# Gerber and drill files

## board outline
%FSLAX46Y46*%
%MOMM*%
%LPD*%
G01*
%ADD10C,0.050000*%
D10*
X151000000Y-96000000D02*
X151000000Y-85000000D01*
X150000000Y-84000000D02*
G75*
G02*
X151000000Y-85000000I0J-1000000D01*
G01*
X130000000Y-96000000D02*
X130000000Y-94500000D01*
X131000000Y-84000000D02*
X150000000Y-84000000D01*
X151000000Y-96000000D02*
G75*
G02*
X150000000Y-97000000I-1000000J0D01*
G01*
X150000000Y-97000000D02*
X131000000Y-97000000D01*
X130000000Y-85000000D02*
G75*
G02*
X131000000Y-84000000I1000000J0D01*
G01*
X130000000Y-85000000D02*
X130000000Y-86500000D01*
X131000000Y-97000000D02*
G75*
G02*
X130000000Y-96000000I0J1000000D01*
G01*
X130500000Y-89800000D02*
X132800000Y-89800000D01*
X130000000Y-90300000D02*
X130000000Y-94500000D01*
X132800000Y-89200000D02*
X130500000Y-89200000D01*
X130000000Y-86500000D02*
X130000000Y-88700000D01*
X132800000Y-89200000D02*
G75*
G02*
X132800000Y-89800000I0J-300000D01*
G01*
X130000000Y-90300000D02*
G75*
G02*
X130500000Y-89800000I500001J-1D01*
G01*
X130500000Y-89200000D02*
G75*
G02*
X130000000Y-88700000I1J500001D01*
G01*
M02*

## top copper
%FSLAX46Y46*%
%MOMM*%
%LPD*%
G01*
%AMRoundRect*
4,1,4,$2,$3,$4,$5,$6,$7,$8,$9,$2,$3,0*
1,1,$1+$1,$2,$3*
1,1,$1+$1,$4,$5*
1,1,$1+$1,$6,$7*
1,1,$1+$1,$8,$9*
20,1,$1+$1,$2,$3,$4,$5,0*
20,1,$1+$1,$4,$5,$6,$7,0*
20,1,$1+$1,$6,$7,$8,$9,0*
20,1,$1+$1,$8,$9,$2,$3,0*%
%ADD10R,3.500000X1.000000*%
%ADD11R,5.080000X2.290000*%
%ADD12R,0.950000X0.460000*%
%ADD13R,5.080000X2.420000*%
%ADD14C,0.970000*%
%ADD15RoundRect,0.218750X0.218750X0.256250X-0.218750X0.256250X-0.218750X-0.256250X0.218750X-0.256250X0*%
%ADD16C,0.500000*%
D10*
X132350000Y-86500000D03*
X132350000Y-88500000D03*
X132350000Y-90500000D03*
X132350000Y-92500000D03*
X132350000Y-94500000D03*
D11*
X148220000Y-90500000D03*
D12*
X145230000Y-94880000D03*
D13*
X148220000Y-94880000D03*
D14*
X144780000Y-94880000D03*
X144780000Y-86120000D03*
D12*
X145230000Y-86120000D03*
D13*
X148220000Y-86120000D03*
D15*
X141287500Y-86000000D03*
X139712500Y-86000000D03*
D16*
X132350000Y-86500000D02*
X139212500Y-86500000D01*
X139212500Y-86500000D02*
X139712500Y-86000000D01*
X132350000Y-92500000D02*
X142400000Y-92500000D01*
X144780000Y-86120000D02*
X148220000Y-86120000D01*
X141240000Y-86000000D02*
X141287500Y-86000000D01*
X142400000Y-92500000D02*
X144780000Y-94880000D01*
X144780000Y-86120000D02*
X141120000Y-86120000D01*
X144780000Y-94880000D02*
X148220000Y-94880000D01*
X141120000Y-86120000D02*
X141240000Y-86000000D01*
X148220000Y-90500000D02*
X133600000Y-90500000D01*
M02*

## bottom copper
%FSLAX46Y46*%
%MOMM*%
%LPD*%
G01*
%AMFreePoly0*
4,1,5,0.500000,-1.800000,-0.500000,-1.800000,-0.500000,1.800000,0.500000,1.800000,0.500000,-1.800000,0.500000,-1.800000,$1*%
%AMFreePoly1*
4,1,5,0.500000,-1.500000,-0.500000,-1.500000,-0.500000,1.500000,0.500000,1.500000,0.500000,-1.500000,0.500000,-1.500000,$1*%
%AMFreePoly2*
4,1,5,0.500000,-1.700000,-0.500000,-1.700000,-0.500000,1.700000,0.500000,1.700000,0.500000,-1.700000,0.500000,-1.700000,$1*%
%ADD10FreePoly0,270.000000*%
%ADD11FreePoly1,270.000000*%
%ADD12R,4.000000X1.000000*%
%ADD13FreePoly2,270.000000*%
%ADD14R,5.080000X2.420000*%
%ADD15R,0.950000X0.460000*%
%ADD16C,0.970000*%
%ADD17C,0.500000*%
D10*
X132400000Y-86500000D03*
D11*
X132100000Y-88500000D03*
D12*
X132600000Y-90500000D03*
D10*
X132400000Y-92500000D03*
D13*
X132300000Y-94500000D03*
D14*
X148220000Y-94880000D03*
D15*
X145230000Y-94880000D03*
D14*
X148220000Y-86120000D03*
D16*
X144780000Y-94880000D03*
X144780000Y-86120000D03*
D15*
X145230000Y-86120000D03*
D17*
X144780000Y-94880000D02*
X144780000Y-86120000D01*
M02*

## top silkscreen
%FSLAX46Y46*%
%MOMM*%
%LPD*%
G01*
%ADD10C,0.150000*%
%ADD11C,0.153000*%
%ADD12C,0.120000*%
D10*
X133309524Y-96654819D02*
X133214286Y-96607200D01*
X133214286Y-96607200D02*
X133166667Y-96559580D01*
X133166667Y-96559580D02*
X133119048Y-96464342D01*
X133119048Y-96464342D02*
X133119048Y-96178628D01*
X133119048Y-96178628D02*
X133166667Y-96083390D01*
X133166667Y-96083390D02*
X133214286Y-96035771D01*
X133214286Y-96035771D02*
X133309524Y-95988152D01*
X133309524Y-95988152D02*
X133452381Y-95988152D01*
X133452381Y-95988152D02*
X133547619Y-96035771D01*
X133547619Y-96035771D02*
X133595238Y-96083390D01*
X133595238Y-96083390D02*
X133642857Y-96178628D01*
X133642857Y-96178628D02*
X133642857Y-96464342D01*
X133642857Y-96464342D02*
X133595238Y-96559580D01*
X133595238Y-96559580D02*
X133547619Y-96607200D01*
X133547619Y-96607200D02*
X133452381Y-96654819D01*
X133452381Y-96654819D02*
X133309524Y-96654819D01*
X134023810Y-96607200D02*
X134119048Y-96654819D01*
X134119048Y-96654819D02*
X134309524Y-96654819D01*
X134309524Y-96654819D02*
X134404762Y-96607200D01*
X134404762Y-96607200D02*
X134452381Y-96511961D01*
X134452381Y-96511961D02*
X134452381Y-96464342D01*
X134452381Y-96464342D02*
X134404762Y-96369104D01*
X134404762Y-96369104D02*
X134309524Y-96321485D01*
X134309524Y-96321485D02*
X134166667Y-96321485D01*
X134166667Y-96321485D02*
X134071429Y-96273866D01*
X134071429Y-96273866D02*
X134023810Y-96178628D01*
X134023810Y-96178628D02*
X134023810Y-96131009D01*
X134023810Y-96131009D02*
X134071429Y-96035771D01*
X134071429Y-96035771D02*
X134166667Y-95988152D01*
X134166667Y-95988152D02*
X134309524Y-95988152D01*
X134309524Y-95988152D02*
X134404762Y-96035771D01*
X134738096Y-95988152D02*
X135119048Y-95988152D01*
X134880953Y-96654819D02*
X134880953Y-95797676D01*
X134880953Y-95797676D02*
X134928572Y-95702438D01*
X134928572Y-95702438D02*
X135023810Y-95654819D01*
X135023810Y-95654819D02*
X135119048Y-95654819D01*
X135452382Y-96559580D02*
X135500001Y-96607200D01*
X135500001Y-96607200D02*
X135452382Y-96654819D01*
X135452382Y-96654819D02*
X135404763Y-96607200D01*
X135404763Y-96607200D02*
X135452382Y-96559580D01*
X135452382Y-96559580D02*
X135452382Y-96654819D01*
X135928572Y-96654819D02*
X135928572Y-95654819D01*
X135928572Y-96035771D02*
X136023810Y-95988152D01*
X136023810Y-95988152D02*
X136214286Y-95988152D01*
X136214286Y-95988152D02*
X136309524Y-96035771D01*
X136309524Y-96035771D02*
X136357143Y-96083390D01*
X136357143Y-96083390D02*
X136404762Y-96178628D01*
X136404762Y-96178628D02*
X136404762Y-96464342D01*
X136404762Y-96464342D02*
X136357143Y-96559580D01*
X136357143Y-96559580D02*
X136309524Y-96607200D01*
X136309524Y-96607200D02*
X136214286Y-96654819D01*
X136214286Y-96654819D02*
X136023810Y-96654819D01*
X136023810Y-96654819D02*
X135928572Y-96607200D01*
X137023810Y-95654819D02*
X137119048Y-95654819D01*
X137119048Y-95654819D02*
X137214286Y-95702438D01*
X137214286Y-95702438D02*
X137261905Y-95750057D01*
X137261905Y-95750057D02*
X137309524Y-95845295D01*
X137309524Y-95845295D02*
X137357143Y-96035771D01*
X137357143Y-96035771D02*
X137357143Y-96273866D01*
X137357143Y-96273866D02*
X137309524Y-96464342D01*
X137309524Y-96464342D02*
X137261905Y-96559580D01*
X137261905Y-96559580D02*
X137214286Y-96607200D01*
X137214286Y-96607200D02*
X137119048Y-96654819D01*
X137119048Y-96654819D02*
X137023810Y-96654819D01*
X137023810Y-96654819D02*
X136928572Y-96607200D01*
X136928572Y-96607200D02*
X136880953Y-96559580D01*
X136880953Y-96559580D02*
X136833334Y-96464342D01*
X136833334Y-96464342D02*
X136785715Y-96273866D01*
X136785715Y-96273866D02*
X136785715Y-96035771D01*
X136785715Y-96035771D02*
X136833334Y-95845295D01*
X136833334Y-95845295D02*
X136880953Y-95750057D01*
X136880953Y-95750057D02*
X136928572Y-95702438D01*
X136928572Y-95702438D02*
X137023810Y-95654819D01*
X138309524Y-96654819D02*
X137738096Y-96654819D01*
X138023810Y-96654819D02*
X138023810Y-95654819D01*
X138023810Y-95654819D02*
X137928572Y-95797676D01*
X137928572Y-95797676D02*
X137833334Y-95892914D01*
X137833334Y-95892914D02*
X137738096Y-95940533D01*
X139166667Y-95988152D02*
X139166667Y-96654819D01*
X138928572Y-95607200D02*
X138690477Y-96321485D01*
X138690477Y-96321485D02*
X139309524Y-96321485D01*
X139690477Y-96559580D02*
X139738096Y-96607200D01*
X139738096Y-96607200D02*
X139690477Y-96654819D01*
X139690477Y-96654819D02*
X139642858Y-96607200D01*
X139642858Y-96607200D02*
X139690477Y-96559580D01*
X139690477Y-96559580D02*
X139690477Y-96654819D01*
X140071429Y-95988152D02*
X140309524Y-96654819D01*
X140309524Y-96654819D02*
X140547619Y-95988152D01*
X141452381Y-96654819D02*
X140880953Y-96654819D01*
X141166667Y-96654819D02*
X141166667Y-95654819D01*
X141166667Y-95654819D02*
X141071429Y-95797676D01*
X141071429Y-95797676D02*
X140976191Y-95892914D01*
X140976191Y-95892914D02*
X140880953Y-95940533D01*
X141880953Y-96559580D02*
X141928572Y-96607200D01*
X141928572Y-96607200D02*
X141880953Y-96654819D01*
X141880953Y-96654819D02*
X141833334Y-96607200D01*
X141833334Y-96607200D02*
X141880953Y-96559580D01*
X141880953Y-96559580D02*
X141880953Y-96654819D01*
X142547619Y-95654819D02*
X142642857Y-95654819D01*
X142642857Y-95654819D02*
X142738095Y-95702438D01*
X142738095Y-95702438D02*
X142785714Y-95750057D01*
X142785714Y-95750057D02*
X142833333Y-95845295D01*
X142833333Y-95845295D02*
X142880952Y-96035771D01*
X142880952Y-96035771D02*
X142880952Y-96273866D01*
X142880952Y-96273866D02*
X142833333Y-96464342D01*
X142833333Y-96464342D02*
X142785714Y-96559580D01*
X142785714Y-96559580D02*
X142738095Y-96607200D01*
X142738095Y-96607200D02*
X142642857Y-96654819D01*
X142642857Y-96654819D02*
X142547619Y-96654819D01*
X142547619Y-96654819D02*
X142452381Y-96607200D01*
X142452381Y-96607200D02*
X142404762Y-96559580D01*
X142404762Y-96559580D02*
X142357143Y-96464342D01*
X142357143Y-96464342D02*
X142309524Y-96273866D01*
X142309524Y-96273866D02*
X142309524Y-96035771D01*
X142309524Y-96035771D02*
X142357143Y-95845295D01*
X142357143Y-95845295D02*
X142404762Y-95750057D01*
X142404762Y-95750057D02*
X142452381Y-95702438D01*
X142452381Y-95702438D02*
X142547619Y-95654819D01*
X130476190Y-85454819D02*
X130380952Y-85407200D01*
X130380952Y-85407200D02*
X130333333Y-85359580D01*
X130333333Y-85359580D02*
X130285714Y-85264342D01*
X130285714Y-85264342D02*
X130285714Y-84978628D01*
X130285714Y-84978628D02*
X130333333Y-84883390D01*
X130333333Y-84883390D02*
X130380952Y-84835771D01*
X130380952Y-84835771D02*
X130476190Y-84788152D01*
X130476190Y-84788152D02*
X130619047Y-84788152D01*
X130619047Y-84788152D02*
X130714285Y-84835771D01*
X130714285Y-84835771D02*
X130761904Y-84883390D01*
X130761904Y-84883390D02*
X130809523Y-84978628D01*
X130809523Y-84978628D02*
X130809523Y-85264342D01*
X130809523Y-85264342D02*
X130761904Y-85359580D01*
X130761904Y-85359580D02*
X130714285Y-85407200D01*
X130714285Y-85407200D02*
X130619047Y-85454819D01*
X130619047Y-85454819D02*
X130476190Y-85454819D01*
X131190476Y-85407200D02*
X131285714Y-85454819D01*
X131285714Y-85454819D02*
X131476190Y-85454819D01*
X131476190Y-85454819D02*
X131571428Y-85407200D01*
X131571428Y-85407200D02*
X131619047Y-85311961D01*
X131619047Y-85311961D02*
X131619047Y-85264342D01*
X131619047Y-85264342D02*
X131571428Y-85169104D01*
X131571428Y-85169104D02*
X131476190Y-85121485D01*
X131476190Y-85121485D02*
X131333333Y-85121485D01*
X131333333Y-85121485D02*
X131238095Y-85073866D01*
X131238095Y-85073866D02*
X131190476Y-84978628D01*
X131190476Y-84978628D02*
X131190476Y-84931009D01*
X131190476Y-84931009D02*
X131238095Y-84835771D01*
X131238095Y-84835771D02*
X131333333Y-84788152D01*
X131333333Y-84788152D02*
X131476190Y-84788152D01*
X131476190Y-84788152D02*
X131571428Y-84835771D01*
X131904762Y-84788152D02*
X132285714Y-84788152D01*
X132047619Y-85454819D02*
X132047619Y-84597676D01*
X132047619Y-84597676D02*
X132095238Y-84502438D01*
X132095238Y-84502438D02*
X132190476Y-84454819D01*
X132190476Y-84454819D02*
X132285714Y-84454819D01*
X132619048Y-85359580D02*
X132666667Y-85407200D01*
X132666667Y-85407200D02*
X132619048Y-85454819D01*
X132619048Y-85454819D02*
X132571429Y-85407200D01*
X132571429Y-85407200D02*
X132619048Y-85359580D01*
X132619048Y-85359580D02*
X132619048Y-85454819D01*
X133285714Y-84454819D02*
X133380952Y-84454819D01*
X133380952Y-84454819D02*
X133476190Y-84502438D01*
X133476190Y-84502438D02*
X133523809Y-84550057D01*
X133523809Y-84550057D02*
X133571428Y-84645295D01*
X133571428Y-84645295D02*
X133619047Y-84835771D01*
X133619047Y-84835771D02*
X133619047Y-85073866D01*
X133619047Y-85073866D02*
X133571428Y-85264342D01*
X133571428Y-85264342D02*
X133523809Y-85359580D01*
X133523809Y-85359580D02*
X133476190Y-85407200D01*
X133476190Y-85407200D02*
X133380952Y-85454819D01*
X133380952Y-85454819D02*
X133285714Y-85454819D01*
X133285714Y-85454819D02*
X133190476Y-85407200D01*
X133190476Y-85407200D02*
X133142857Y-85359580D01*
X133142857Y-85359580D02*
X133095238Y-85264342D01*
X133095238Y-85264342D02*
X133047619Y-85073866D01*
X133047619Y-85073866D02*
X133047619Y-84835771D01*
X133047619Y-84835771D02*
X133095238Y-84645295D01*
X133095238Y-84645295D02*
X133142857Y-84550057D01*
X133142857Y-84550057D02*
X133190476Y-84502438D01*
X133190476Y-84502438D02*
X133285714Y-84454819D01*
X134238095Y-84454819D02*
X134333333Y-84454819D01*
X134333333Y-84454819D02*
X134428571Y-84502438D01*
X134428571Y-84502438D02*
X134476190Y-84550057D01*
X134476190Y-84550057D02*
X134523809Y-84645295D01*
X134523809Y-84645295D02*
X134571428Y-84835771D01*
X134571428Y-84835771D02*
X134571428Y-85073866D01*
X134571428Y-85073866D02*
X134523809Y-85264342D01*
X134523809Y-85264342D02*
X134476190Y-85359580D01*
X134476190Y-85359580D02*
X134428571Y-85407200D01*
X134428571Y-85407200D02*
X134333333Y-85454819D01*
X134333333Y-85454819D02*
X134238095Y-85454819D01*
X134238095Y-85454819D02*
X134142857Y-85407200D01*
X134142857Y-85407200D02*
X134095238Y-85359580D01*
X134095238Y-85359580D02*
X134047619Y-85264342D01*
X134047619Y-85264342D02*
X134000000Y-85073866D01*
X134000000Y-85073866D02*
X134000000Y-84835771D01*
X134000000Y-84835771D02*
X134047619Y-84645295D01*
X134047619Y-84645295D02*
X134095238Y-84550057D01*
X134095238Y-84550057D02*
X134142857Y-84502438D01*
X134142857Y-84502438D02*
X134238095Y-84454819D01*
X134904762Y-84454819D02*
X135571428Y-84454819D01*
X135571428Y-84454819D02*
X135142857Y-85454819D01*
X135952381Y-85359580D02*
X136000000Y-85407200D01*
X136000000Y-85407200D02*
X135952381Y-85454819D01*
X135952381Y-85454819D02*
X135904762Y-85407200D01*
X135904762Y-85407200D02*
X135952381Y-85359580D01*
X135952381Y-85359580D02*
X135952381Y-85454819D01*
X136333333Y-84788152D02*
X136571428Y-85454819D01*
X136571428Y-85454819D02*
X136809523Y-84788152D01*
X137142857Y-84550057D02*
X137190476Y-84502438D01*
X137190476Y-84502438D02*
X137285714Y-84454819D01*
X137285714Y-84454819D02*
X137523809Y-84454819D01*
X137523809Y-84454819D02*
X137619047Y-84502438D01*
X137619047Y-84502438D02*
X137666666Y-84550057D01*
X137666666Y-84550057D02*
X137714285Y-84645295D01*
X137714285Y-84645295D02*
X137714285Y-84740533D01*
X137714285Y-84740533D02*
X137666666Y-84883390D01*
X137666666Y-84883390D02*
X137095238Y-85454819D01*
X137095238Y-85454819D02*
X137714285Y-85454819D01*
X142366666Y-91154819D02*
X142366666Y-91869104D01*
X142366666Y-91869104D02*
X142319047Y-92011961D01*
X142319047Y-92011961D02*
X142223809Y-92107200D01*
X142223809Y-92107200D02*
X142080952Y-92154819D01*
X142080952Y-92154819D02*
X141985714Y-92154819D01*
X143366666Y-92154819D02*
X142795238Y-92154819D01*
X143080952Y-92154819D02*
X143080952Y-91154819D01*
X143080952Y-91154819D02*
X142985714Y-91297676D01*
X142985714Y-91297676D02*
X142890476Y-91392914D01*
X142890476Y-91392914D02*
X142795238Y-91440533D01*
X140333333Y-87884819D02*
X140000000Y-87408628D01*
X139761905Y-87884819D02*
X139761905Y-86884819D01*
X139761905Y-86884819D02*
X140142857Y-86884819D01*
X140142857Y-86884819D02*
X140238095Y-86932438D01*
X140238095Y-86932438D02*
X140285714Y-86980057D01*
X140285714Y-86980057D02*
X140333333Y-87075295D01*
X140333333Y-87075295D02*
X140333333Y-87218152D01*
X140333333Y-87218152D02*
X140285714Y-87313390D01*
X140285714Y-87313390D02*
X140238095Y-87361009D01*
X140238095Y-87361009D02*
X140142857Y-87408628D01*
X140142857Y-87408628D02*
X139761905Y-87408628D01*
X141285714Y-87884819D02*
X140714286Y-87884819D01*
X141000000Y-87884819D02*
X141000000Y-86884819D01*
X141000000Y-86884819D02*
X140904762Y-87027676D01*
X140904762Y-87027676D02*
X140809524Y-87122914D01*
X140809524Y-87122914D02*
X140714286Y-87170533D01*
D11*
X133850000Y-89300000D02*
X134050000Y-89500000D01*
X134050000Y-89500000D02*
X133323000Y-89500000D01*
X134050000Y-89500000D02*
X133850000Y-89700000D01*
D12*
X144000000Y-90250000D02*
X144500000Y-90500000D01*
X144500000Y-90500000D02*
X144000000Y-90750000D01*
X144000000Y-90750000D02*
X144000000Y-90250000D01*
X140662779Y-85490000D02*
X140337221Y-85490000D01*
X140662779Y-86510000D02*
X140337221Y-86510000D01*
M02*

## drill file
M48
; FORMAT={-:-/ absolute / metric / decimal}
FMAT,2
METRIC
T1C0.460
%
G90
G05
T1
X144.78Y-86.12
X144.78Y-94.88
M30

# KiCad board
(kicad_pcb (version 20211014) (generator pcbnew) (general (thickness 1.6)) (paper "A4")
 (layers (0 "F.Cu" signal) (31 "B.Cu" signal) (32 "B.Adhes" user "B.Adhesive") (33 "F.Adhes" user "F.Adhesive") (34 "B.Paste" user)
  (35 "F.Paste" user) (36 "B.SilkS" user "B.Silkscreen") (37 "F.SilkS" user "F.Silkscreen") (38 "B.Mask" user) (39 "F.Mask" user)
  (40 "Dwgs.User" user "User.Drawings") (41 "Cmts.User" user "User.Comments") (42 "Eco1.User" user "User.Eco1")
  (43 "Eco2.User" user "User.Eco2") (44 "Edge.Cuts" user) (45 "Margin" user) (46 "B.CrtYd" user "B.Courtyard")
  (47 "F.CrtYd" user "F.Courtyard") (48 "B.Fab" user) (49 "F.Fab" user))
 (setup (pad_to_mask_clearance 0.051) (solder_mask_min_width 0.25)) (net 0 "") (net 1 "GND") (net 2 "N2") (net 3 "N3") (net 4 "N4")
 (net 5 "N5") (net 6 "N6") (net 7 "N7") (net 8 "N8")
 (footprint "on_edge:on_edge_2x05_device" (layer "F.Cu") (at 130 90.5 -90)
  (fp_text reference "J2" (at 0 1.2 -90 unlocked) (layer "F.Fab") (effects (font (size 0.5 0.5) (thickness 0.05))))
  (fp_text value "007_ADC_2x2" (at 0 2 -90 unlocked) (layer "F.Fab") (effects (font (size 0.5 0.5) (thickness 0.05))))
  (fp_line (start -1.2 -3.85) (end -1 -4.05) (layer "F.SilkS") (width 0.153))
  (fp_line (start -1 -4.05) (end -1 -3.323) (layer "F.SilkS") (width 0.153))
  (fp_line (start -1 -4.05) (end -0.8 -3.85) (layer "F.SilkS") (width 0.153))
  (fp_line (start -0.7 -0.5) (end -0.7 -2.8) (layer "Edge.Cuts") (width 0.05))
  (fp_line (start -0.2 0) (end 4 0) (layer "Edge.Cuts") (width 0.05))
  (fp_line (start -1.3 -2.8) (end -1.3 -0.5) (layer "Edge.Cuts") (width 0.05))
  (fp_line (start -4 0) (end -1.8 0) (layer "Edge.Cuts") (width 0.05))
  (fp_arc (start -1.3 -2.8) (mid -1 -3.1) (end -0.7 -2.8) (layer "Edge.Cuts") (width 0.05))
  (fp_arc (start -0.2 0) (mid -0.553553 -0.146447) (end -0.7 -0.5) (layer "Edge.Cuts") (width 0.05))
  (fp_arc (start -1.3 -0.5) (mid -1.446447 -0.146447) (end -1.8 0) (layer "Edge.Cuts") (width 0.05))
  (pad "1" smd rect (at -4 -2.35 90) (size 1 3.5) (layers "F.Cu" "F.Mask") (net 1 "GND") (zone_connect 0))
  (pad "2" smd rect (at -2 -2.35 270) (size 1 3.5) (layers "F.Cu" "F.Mask") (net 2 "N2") (zone_connect 0))
  (pad "3" smd rect (at 0 -2.35 270) (size 1 3.5) (layers "F.Cu" "F.Mask") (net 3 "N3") (zone_connect 0))
  (pad "4" smd rect (at 2 -2.35 90) (size 1 3.5) (layers "F.Cu" "F.Mask") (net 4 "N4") (zone_connect 0))
  (pad "5" smd rect (at 4 -2.35 90) (size 1 3.5) (layers "F.Cu" "F.Mask") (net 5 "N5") (zone_connect 0))
  (pad "6" smd custom (at -4 -2.4 270) (size 1 3.6) (layers "B.Cu" "B.Mask") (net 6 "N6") (zone_connect 0)
   (options (clearance outline) (anchor rect)) (primitives))
  (pad "7" smd custom (at -2 -2.1 270) (size 1 3) (layers "B.Cu" "B.Mask") (zone_connect 0) (options (clearance outline) (anchor rect))
   (primitives))
  (pad "8" smd rect (at 0 -2.6 270) (size 1 4) (layers "B.Cu" "B.Mask") (zone_connect 0))
  (pad "9" smd custom (at 2 -2.4 270) (size 1 3.6) (layers "B.Cu" "B.Mask") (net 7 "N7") (zone_connect 0)
   (options (clearance outline) (anchor rect)) (primitives))
  (pad "10" smd custom (at 4 -2.3 270) (size 1 3.4) (layers "B.Cu" "B.Mask") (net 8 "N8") (zone_connect 0)
   (options (clearance outline) (anchor rect)) (primitives)))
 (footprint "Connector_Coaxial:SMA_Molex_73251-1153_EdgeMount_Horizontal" (layer "F.Cu") (at 146.5 90.5 180)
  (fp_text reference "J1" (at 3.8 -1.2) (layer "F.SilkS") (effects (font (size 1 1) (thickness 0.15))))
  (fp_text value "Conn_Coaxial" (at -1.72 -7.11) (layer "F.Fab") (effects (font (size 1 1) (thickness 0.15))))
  (fp_line (start 2.5 0.25) (end 2 0) (layer "F.SilkS") (width 0.12))
  (fp_line (start 2 0) (end 2.5 -0.25) (layer "F.SilkS") (width 0.12))
  (fp_line (start 2.5 -0.25) (end 2.5 0.25) (layer "F.SilkS") (width 0.12))
  (pad "1" smd rect locked (at -1.72 0 180) (size 5.08 2.29) (layers "F.Cu" "F.Paste" "F.Mask") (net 3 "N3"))
  (pad "2" smd rect locked (at 1.27 -4.38 180) (size 0.95 0.46) (layers "F.Cu") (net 4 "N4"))
  (pad "2" smd rect locked (at -1.72 -4.38 180) (size 5.08 2.42) (layers "B.Cu" "B.Paste" "B.Mask") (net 4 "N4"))
  (pad "2" smd rect locked (at -1.72 -4.38 180) (size 5.08 2.42) (layers "F.Cu" "F.Paste" "F.Mask") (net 4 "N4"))
  (pad "2" smd rect locked (at 1.27 -4.38 180) (size 0.95 0.46) (layers "B.Cu") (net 4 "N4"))
  (pad "2" smd rect locked (at -1.72 4.38 180) (size 5.08 2.42) (layers "B.Cu" "B.Paste" "B.Mask") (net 4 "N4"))
  (pad "2" thru_hole circle locked (at 1.72 -4.38 180) (size 0.97 0.97) (drill 0.46) (layers *.Cu) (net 4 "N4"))
  (pad "2" thru_hole circle locked (at 1.72 4.38 180) (size 0.97 0.97) (drill 0.46) (layers *.Cu) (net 4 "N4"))
  (pad "2" smd rect locked (at 1.27 4.38 180) (size 0.95 0.46) (layers "B.Cu") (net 4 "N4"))
  (pad "2" smd rect locked (at 1.27 4.38 180) (size 0.95 0.46) (layers "F.Cu") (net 4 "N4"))
  (pad "2" smd rect locked (at -1.72 4.38 180) (size 5.08 2.42) (layers "F.Cu" "F.Paste" "F.Mask") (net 4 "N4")))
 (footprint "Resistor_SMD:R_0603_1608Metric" (layer "F.Cu") (at 140.5 86 180)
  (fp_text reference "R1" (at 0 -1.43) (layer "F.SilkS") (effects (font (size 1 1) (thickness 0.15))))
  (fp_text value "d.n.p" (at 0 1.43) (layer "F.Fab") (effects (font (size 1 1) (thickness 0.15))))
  (fp_line (start -0.162779 0.51) (end 0.162779 0.51) (layer "F.SilkS") (width 0.12))
  (fp_line (start -0.162779 -0.51) (end 0.162779 -0.51) (layer "F.SilkS") (width 0.12))
  (pad "1" smd roundrect locked (at -0.7875 0 180) (size 0.875 0.95) (layers "F.Cu" "F.Paste" "F.Mask") (roundrect_rratio 0.25) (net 4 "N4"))
  (pad "2" smd roundrect locked (at 0.7875 0 180) (size 0.875 0.95) (layers "F.Cu" "F.Paste" "F.Mask") (roundrect_rratio 0.25) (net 1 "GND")))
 (gr_line (start 151 96) (end 151 85) (layer "Edge.Cuts") (width 0.05))
 (gr_arc (start 150 84) (mid 150.707107 84.292893) (end 151 85) (layer "Edge.Cuts") (width 0.05))
 (gr_line (start 130 96) (end 130 94.5) (layer "Edge.Cuts") (width 0.05))
 (gr_line (start 131 84) (end 150 84) (layer "Edge.Cuts") (width 0.05))
 (gr_arc (start 151 96) (mid 150.707107 96.707107) (end 150 97) (layer "Edge.Cuts") (width 0.05))
 (gr_line (start 150 97) (end 131 97) (layer "Edge.Cuts") (width 0.05))
 (gr_arc (start 130 85) (mid 130.292893 84.292893) (end 131 84) (layer "Edge.Cuts") (width 0.05))
 (gr_line (start 130 85) (end 130 86.5) (layer "Edge.Cuts") (width 0.05))
 (gr_arc (start 131 97) (mid 130.292893 96.707107) (end 130 96) (layer "Edge.Cuts") (width 0.05))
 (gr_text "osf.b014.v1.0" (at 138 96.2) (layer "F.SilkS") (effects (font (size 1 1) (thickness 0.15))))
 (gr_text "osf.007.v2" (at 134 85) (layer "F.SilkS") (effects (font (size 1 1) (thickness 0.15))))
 (segment (start 132.35 86.5) (end 139.2125 86.5) (width 0.5) (layer "F.Cu") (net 1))
 (segment (start 139.2125 86.5) (end 139.7125 86) (width 0.5) (layer "F.Cu") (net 1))
 (segment (start 132.35 92.5) (end 142.4 92.5) (width 0.5) (layer "F.Cu") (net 4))
 (segment (start 144.78 86.12) (end 148.22 86.12) (width 0.5) (layer "F.Cu") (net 4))
 (segment (start 141.24 86) (end 141.2875 86) (width 0.5) (layer "F.Cu") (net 4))
 (segment (start 142.4 92.5) (end 144.78 94.88) (width 0.5) (layer "F.Cu") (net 4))
 (segment (start 144.78 86.12) (end 141.12 86.12) (width 0.5) (layer "F.Cu") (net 4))
 (segment (start 144.78 94.88) (end 148.22 94.88) (width 0.5) (layer "F.Cu") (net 4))
 (segment (start 141.12 86.12) (end 141.24 86) (width 0.5) (layer "F.Cu") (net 4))
 (segment (start 144.78 94.88) (end 144.78 86.12) (width 0.5) (layer "B.Cu") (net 4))
 (segment (start 148.22 90.5) (end 133.6 90.5) (width 0.5) (layer "F.Cu") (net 3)))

